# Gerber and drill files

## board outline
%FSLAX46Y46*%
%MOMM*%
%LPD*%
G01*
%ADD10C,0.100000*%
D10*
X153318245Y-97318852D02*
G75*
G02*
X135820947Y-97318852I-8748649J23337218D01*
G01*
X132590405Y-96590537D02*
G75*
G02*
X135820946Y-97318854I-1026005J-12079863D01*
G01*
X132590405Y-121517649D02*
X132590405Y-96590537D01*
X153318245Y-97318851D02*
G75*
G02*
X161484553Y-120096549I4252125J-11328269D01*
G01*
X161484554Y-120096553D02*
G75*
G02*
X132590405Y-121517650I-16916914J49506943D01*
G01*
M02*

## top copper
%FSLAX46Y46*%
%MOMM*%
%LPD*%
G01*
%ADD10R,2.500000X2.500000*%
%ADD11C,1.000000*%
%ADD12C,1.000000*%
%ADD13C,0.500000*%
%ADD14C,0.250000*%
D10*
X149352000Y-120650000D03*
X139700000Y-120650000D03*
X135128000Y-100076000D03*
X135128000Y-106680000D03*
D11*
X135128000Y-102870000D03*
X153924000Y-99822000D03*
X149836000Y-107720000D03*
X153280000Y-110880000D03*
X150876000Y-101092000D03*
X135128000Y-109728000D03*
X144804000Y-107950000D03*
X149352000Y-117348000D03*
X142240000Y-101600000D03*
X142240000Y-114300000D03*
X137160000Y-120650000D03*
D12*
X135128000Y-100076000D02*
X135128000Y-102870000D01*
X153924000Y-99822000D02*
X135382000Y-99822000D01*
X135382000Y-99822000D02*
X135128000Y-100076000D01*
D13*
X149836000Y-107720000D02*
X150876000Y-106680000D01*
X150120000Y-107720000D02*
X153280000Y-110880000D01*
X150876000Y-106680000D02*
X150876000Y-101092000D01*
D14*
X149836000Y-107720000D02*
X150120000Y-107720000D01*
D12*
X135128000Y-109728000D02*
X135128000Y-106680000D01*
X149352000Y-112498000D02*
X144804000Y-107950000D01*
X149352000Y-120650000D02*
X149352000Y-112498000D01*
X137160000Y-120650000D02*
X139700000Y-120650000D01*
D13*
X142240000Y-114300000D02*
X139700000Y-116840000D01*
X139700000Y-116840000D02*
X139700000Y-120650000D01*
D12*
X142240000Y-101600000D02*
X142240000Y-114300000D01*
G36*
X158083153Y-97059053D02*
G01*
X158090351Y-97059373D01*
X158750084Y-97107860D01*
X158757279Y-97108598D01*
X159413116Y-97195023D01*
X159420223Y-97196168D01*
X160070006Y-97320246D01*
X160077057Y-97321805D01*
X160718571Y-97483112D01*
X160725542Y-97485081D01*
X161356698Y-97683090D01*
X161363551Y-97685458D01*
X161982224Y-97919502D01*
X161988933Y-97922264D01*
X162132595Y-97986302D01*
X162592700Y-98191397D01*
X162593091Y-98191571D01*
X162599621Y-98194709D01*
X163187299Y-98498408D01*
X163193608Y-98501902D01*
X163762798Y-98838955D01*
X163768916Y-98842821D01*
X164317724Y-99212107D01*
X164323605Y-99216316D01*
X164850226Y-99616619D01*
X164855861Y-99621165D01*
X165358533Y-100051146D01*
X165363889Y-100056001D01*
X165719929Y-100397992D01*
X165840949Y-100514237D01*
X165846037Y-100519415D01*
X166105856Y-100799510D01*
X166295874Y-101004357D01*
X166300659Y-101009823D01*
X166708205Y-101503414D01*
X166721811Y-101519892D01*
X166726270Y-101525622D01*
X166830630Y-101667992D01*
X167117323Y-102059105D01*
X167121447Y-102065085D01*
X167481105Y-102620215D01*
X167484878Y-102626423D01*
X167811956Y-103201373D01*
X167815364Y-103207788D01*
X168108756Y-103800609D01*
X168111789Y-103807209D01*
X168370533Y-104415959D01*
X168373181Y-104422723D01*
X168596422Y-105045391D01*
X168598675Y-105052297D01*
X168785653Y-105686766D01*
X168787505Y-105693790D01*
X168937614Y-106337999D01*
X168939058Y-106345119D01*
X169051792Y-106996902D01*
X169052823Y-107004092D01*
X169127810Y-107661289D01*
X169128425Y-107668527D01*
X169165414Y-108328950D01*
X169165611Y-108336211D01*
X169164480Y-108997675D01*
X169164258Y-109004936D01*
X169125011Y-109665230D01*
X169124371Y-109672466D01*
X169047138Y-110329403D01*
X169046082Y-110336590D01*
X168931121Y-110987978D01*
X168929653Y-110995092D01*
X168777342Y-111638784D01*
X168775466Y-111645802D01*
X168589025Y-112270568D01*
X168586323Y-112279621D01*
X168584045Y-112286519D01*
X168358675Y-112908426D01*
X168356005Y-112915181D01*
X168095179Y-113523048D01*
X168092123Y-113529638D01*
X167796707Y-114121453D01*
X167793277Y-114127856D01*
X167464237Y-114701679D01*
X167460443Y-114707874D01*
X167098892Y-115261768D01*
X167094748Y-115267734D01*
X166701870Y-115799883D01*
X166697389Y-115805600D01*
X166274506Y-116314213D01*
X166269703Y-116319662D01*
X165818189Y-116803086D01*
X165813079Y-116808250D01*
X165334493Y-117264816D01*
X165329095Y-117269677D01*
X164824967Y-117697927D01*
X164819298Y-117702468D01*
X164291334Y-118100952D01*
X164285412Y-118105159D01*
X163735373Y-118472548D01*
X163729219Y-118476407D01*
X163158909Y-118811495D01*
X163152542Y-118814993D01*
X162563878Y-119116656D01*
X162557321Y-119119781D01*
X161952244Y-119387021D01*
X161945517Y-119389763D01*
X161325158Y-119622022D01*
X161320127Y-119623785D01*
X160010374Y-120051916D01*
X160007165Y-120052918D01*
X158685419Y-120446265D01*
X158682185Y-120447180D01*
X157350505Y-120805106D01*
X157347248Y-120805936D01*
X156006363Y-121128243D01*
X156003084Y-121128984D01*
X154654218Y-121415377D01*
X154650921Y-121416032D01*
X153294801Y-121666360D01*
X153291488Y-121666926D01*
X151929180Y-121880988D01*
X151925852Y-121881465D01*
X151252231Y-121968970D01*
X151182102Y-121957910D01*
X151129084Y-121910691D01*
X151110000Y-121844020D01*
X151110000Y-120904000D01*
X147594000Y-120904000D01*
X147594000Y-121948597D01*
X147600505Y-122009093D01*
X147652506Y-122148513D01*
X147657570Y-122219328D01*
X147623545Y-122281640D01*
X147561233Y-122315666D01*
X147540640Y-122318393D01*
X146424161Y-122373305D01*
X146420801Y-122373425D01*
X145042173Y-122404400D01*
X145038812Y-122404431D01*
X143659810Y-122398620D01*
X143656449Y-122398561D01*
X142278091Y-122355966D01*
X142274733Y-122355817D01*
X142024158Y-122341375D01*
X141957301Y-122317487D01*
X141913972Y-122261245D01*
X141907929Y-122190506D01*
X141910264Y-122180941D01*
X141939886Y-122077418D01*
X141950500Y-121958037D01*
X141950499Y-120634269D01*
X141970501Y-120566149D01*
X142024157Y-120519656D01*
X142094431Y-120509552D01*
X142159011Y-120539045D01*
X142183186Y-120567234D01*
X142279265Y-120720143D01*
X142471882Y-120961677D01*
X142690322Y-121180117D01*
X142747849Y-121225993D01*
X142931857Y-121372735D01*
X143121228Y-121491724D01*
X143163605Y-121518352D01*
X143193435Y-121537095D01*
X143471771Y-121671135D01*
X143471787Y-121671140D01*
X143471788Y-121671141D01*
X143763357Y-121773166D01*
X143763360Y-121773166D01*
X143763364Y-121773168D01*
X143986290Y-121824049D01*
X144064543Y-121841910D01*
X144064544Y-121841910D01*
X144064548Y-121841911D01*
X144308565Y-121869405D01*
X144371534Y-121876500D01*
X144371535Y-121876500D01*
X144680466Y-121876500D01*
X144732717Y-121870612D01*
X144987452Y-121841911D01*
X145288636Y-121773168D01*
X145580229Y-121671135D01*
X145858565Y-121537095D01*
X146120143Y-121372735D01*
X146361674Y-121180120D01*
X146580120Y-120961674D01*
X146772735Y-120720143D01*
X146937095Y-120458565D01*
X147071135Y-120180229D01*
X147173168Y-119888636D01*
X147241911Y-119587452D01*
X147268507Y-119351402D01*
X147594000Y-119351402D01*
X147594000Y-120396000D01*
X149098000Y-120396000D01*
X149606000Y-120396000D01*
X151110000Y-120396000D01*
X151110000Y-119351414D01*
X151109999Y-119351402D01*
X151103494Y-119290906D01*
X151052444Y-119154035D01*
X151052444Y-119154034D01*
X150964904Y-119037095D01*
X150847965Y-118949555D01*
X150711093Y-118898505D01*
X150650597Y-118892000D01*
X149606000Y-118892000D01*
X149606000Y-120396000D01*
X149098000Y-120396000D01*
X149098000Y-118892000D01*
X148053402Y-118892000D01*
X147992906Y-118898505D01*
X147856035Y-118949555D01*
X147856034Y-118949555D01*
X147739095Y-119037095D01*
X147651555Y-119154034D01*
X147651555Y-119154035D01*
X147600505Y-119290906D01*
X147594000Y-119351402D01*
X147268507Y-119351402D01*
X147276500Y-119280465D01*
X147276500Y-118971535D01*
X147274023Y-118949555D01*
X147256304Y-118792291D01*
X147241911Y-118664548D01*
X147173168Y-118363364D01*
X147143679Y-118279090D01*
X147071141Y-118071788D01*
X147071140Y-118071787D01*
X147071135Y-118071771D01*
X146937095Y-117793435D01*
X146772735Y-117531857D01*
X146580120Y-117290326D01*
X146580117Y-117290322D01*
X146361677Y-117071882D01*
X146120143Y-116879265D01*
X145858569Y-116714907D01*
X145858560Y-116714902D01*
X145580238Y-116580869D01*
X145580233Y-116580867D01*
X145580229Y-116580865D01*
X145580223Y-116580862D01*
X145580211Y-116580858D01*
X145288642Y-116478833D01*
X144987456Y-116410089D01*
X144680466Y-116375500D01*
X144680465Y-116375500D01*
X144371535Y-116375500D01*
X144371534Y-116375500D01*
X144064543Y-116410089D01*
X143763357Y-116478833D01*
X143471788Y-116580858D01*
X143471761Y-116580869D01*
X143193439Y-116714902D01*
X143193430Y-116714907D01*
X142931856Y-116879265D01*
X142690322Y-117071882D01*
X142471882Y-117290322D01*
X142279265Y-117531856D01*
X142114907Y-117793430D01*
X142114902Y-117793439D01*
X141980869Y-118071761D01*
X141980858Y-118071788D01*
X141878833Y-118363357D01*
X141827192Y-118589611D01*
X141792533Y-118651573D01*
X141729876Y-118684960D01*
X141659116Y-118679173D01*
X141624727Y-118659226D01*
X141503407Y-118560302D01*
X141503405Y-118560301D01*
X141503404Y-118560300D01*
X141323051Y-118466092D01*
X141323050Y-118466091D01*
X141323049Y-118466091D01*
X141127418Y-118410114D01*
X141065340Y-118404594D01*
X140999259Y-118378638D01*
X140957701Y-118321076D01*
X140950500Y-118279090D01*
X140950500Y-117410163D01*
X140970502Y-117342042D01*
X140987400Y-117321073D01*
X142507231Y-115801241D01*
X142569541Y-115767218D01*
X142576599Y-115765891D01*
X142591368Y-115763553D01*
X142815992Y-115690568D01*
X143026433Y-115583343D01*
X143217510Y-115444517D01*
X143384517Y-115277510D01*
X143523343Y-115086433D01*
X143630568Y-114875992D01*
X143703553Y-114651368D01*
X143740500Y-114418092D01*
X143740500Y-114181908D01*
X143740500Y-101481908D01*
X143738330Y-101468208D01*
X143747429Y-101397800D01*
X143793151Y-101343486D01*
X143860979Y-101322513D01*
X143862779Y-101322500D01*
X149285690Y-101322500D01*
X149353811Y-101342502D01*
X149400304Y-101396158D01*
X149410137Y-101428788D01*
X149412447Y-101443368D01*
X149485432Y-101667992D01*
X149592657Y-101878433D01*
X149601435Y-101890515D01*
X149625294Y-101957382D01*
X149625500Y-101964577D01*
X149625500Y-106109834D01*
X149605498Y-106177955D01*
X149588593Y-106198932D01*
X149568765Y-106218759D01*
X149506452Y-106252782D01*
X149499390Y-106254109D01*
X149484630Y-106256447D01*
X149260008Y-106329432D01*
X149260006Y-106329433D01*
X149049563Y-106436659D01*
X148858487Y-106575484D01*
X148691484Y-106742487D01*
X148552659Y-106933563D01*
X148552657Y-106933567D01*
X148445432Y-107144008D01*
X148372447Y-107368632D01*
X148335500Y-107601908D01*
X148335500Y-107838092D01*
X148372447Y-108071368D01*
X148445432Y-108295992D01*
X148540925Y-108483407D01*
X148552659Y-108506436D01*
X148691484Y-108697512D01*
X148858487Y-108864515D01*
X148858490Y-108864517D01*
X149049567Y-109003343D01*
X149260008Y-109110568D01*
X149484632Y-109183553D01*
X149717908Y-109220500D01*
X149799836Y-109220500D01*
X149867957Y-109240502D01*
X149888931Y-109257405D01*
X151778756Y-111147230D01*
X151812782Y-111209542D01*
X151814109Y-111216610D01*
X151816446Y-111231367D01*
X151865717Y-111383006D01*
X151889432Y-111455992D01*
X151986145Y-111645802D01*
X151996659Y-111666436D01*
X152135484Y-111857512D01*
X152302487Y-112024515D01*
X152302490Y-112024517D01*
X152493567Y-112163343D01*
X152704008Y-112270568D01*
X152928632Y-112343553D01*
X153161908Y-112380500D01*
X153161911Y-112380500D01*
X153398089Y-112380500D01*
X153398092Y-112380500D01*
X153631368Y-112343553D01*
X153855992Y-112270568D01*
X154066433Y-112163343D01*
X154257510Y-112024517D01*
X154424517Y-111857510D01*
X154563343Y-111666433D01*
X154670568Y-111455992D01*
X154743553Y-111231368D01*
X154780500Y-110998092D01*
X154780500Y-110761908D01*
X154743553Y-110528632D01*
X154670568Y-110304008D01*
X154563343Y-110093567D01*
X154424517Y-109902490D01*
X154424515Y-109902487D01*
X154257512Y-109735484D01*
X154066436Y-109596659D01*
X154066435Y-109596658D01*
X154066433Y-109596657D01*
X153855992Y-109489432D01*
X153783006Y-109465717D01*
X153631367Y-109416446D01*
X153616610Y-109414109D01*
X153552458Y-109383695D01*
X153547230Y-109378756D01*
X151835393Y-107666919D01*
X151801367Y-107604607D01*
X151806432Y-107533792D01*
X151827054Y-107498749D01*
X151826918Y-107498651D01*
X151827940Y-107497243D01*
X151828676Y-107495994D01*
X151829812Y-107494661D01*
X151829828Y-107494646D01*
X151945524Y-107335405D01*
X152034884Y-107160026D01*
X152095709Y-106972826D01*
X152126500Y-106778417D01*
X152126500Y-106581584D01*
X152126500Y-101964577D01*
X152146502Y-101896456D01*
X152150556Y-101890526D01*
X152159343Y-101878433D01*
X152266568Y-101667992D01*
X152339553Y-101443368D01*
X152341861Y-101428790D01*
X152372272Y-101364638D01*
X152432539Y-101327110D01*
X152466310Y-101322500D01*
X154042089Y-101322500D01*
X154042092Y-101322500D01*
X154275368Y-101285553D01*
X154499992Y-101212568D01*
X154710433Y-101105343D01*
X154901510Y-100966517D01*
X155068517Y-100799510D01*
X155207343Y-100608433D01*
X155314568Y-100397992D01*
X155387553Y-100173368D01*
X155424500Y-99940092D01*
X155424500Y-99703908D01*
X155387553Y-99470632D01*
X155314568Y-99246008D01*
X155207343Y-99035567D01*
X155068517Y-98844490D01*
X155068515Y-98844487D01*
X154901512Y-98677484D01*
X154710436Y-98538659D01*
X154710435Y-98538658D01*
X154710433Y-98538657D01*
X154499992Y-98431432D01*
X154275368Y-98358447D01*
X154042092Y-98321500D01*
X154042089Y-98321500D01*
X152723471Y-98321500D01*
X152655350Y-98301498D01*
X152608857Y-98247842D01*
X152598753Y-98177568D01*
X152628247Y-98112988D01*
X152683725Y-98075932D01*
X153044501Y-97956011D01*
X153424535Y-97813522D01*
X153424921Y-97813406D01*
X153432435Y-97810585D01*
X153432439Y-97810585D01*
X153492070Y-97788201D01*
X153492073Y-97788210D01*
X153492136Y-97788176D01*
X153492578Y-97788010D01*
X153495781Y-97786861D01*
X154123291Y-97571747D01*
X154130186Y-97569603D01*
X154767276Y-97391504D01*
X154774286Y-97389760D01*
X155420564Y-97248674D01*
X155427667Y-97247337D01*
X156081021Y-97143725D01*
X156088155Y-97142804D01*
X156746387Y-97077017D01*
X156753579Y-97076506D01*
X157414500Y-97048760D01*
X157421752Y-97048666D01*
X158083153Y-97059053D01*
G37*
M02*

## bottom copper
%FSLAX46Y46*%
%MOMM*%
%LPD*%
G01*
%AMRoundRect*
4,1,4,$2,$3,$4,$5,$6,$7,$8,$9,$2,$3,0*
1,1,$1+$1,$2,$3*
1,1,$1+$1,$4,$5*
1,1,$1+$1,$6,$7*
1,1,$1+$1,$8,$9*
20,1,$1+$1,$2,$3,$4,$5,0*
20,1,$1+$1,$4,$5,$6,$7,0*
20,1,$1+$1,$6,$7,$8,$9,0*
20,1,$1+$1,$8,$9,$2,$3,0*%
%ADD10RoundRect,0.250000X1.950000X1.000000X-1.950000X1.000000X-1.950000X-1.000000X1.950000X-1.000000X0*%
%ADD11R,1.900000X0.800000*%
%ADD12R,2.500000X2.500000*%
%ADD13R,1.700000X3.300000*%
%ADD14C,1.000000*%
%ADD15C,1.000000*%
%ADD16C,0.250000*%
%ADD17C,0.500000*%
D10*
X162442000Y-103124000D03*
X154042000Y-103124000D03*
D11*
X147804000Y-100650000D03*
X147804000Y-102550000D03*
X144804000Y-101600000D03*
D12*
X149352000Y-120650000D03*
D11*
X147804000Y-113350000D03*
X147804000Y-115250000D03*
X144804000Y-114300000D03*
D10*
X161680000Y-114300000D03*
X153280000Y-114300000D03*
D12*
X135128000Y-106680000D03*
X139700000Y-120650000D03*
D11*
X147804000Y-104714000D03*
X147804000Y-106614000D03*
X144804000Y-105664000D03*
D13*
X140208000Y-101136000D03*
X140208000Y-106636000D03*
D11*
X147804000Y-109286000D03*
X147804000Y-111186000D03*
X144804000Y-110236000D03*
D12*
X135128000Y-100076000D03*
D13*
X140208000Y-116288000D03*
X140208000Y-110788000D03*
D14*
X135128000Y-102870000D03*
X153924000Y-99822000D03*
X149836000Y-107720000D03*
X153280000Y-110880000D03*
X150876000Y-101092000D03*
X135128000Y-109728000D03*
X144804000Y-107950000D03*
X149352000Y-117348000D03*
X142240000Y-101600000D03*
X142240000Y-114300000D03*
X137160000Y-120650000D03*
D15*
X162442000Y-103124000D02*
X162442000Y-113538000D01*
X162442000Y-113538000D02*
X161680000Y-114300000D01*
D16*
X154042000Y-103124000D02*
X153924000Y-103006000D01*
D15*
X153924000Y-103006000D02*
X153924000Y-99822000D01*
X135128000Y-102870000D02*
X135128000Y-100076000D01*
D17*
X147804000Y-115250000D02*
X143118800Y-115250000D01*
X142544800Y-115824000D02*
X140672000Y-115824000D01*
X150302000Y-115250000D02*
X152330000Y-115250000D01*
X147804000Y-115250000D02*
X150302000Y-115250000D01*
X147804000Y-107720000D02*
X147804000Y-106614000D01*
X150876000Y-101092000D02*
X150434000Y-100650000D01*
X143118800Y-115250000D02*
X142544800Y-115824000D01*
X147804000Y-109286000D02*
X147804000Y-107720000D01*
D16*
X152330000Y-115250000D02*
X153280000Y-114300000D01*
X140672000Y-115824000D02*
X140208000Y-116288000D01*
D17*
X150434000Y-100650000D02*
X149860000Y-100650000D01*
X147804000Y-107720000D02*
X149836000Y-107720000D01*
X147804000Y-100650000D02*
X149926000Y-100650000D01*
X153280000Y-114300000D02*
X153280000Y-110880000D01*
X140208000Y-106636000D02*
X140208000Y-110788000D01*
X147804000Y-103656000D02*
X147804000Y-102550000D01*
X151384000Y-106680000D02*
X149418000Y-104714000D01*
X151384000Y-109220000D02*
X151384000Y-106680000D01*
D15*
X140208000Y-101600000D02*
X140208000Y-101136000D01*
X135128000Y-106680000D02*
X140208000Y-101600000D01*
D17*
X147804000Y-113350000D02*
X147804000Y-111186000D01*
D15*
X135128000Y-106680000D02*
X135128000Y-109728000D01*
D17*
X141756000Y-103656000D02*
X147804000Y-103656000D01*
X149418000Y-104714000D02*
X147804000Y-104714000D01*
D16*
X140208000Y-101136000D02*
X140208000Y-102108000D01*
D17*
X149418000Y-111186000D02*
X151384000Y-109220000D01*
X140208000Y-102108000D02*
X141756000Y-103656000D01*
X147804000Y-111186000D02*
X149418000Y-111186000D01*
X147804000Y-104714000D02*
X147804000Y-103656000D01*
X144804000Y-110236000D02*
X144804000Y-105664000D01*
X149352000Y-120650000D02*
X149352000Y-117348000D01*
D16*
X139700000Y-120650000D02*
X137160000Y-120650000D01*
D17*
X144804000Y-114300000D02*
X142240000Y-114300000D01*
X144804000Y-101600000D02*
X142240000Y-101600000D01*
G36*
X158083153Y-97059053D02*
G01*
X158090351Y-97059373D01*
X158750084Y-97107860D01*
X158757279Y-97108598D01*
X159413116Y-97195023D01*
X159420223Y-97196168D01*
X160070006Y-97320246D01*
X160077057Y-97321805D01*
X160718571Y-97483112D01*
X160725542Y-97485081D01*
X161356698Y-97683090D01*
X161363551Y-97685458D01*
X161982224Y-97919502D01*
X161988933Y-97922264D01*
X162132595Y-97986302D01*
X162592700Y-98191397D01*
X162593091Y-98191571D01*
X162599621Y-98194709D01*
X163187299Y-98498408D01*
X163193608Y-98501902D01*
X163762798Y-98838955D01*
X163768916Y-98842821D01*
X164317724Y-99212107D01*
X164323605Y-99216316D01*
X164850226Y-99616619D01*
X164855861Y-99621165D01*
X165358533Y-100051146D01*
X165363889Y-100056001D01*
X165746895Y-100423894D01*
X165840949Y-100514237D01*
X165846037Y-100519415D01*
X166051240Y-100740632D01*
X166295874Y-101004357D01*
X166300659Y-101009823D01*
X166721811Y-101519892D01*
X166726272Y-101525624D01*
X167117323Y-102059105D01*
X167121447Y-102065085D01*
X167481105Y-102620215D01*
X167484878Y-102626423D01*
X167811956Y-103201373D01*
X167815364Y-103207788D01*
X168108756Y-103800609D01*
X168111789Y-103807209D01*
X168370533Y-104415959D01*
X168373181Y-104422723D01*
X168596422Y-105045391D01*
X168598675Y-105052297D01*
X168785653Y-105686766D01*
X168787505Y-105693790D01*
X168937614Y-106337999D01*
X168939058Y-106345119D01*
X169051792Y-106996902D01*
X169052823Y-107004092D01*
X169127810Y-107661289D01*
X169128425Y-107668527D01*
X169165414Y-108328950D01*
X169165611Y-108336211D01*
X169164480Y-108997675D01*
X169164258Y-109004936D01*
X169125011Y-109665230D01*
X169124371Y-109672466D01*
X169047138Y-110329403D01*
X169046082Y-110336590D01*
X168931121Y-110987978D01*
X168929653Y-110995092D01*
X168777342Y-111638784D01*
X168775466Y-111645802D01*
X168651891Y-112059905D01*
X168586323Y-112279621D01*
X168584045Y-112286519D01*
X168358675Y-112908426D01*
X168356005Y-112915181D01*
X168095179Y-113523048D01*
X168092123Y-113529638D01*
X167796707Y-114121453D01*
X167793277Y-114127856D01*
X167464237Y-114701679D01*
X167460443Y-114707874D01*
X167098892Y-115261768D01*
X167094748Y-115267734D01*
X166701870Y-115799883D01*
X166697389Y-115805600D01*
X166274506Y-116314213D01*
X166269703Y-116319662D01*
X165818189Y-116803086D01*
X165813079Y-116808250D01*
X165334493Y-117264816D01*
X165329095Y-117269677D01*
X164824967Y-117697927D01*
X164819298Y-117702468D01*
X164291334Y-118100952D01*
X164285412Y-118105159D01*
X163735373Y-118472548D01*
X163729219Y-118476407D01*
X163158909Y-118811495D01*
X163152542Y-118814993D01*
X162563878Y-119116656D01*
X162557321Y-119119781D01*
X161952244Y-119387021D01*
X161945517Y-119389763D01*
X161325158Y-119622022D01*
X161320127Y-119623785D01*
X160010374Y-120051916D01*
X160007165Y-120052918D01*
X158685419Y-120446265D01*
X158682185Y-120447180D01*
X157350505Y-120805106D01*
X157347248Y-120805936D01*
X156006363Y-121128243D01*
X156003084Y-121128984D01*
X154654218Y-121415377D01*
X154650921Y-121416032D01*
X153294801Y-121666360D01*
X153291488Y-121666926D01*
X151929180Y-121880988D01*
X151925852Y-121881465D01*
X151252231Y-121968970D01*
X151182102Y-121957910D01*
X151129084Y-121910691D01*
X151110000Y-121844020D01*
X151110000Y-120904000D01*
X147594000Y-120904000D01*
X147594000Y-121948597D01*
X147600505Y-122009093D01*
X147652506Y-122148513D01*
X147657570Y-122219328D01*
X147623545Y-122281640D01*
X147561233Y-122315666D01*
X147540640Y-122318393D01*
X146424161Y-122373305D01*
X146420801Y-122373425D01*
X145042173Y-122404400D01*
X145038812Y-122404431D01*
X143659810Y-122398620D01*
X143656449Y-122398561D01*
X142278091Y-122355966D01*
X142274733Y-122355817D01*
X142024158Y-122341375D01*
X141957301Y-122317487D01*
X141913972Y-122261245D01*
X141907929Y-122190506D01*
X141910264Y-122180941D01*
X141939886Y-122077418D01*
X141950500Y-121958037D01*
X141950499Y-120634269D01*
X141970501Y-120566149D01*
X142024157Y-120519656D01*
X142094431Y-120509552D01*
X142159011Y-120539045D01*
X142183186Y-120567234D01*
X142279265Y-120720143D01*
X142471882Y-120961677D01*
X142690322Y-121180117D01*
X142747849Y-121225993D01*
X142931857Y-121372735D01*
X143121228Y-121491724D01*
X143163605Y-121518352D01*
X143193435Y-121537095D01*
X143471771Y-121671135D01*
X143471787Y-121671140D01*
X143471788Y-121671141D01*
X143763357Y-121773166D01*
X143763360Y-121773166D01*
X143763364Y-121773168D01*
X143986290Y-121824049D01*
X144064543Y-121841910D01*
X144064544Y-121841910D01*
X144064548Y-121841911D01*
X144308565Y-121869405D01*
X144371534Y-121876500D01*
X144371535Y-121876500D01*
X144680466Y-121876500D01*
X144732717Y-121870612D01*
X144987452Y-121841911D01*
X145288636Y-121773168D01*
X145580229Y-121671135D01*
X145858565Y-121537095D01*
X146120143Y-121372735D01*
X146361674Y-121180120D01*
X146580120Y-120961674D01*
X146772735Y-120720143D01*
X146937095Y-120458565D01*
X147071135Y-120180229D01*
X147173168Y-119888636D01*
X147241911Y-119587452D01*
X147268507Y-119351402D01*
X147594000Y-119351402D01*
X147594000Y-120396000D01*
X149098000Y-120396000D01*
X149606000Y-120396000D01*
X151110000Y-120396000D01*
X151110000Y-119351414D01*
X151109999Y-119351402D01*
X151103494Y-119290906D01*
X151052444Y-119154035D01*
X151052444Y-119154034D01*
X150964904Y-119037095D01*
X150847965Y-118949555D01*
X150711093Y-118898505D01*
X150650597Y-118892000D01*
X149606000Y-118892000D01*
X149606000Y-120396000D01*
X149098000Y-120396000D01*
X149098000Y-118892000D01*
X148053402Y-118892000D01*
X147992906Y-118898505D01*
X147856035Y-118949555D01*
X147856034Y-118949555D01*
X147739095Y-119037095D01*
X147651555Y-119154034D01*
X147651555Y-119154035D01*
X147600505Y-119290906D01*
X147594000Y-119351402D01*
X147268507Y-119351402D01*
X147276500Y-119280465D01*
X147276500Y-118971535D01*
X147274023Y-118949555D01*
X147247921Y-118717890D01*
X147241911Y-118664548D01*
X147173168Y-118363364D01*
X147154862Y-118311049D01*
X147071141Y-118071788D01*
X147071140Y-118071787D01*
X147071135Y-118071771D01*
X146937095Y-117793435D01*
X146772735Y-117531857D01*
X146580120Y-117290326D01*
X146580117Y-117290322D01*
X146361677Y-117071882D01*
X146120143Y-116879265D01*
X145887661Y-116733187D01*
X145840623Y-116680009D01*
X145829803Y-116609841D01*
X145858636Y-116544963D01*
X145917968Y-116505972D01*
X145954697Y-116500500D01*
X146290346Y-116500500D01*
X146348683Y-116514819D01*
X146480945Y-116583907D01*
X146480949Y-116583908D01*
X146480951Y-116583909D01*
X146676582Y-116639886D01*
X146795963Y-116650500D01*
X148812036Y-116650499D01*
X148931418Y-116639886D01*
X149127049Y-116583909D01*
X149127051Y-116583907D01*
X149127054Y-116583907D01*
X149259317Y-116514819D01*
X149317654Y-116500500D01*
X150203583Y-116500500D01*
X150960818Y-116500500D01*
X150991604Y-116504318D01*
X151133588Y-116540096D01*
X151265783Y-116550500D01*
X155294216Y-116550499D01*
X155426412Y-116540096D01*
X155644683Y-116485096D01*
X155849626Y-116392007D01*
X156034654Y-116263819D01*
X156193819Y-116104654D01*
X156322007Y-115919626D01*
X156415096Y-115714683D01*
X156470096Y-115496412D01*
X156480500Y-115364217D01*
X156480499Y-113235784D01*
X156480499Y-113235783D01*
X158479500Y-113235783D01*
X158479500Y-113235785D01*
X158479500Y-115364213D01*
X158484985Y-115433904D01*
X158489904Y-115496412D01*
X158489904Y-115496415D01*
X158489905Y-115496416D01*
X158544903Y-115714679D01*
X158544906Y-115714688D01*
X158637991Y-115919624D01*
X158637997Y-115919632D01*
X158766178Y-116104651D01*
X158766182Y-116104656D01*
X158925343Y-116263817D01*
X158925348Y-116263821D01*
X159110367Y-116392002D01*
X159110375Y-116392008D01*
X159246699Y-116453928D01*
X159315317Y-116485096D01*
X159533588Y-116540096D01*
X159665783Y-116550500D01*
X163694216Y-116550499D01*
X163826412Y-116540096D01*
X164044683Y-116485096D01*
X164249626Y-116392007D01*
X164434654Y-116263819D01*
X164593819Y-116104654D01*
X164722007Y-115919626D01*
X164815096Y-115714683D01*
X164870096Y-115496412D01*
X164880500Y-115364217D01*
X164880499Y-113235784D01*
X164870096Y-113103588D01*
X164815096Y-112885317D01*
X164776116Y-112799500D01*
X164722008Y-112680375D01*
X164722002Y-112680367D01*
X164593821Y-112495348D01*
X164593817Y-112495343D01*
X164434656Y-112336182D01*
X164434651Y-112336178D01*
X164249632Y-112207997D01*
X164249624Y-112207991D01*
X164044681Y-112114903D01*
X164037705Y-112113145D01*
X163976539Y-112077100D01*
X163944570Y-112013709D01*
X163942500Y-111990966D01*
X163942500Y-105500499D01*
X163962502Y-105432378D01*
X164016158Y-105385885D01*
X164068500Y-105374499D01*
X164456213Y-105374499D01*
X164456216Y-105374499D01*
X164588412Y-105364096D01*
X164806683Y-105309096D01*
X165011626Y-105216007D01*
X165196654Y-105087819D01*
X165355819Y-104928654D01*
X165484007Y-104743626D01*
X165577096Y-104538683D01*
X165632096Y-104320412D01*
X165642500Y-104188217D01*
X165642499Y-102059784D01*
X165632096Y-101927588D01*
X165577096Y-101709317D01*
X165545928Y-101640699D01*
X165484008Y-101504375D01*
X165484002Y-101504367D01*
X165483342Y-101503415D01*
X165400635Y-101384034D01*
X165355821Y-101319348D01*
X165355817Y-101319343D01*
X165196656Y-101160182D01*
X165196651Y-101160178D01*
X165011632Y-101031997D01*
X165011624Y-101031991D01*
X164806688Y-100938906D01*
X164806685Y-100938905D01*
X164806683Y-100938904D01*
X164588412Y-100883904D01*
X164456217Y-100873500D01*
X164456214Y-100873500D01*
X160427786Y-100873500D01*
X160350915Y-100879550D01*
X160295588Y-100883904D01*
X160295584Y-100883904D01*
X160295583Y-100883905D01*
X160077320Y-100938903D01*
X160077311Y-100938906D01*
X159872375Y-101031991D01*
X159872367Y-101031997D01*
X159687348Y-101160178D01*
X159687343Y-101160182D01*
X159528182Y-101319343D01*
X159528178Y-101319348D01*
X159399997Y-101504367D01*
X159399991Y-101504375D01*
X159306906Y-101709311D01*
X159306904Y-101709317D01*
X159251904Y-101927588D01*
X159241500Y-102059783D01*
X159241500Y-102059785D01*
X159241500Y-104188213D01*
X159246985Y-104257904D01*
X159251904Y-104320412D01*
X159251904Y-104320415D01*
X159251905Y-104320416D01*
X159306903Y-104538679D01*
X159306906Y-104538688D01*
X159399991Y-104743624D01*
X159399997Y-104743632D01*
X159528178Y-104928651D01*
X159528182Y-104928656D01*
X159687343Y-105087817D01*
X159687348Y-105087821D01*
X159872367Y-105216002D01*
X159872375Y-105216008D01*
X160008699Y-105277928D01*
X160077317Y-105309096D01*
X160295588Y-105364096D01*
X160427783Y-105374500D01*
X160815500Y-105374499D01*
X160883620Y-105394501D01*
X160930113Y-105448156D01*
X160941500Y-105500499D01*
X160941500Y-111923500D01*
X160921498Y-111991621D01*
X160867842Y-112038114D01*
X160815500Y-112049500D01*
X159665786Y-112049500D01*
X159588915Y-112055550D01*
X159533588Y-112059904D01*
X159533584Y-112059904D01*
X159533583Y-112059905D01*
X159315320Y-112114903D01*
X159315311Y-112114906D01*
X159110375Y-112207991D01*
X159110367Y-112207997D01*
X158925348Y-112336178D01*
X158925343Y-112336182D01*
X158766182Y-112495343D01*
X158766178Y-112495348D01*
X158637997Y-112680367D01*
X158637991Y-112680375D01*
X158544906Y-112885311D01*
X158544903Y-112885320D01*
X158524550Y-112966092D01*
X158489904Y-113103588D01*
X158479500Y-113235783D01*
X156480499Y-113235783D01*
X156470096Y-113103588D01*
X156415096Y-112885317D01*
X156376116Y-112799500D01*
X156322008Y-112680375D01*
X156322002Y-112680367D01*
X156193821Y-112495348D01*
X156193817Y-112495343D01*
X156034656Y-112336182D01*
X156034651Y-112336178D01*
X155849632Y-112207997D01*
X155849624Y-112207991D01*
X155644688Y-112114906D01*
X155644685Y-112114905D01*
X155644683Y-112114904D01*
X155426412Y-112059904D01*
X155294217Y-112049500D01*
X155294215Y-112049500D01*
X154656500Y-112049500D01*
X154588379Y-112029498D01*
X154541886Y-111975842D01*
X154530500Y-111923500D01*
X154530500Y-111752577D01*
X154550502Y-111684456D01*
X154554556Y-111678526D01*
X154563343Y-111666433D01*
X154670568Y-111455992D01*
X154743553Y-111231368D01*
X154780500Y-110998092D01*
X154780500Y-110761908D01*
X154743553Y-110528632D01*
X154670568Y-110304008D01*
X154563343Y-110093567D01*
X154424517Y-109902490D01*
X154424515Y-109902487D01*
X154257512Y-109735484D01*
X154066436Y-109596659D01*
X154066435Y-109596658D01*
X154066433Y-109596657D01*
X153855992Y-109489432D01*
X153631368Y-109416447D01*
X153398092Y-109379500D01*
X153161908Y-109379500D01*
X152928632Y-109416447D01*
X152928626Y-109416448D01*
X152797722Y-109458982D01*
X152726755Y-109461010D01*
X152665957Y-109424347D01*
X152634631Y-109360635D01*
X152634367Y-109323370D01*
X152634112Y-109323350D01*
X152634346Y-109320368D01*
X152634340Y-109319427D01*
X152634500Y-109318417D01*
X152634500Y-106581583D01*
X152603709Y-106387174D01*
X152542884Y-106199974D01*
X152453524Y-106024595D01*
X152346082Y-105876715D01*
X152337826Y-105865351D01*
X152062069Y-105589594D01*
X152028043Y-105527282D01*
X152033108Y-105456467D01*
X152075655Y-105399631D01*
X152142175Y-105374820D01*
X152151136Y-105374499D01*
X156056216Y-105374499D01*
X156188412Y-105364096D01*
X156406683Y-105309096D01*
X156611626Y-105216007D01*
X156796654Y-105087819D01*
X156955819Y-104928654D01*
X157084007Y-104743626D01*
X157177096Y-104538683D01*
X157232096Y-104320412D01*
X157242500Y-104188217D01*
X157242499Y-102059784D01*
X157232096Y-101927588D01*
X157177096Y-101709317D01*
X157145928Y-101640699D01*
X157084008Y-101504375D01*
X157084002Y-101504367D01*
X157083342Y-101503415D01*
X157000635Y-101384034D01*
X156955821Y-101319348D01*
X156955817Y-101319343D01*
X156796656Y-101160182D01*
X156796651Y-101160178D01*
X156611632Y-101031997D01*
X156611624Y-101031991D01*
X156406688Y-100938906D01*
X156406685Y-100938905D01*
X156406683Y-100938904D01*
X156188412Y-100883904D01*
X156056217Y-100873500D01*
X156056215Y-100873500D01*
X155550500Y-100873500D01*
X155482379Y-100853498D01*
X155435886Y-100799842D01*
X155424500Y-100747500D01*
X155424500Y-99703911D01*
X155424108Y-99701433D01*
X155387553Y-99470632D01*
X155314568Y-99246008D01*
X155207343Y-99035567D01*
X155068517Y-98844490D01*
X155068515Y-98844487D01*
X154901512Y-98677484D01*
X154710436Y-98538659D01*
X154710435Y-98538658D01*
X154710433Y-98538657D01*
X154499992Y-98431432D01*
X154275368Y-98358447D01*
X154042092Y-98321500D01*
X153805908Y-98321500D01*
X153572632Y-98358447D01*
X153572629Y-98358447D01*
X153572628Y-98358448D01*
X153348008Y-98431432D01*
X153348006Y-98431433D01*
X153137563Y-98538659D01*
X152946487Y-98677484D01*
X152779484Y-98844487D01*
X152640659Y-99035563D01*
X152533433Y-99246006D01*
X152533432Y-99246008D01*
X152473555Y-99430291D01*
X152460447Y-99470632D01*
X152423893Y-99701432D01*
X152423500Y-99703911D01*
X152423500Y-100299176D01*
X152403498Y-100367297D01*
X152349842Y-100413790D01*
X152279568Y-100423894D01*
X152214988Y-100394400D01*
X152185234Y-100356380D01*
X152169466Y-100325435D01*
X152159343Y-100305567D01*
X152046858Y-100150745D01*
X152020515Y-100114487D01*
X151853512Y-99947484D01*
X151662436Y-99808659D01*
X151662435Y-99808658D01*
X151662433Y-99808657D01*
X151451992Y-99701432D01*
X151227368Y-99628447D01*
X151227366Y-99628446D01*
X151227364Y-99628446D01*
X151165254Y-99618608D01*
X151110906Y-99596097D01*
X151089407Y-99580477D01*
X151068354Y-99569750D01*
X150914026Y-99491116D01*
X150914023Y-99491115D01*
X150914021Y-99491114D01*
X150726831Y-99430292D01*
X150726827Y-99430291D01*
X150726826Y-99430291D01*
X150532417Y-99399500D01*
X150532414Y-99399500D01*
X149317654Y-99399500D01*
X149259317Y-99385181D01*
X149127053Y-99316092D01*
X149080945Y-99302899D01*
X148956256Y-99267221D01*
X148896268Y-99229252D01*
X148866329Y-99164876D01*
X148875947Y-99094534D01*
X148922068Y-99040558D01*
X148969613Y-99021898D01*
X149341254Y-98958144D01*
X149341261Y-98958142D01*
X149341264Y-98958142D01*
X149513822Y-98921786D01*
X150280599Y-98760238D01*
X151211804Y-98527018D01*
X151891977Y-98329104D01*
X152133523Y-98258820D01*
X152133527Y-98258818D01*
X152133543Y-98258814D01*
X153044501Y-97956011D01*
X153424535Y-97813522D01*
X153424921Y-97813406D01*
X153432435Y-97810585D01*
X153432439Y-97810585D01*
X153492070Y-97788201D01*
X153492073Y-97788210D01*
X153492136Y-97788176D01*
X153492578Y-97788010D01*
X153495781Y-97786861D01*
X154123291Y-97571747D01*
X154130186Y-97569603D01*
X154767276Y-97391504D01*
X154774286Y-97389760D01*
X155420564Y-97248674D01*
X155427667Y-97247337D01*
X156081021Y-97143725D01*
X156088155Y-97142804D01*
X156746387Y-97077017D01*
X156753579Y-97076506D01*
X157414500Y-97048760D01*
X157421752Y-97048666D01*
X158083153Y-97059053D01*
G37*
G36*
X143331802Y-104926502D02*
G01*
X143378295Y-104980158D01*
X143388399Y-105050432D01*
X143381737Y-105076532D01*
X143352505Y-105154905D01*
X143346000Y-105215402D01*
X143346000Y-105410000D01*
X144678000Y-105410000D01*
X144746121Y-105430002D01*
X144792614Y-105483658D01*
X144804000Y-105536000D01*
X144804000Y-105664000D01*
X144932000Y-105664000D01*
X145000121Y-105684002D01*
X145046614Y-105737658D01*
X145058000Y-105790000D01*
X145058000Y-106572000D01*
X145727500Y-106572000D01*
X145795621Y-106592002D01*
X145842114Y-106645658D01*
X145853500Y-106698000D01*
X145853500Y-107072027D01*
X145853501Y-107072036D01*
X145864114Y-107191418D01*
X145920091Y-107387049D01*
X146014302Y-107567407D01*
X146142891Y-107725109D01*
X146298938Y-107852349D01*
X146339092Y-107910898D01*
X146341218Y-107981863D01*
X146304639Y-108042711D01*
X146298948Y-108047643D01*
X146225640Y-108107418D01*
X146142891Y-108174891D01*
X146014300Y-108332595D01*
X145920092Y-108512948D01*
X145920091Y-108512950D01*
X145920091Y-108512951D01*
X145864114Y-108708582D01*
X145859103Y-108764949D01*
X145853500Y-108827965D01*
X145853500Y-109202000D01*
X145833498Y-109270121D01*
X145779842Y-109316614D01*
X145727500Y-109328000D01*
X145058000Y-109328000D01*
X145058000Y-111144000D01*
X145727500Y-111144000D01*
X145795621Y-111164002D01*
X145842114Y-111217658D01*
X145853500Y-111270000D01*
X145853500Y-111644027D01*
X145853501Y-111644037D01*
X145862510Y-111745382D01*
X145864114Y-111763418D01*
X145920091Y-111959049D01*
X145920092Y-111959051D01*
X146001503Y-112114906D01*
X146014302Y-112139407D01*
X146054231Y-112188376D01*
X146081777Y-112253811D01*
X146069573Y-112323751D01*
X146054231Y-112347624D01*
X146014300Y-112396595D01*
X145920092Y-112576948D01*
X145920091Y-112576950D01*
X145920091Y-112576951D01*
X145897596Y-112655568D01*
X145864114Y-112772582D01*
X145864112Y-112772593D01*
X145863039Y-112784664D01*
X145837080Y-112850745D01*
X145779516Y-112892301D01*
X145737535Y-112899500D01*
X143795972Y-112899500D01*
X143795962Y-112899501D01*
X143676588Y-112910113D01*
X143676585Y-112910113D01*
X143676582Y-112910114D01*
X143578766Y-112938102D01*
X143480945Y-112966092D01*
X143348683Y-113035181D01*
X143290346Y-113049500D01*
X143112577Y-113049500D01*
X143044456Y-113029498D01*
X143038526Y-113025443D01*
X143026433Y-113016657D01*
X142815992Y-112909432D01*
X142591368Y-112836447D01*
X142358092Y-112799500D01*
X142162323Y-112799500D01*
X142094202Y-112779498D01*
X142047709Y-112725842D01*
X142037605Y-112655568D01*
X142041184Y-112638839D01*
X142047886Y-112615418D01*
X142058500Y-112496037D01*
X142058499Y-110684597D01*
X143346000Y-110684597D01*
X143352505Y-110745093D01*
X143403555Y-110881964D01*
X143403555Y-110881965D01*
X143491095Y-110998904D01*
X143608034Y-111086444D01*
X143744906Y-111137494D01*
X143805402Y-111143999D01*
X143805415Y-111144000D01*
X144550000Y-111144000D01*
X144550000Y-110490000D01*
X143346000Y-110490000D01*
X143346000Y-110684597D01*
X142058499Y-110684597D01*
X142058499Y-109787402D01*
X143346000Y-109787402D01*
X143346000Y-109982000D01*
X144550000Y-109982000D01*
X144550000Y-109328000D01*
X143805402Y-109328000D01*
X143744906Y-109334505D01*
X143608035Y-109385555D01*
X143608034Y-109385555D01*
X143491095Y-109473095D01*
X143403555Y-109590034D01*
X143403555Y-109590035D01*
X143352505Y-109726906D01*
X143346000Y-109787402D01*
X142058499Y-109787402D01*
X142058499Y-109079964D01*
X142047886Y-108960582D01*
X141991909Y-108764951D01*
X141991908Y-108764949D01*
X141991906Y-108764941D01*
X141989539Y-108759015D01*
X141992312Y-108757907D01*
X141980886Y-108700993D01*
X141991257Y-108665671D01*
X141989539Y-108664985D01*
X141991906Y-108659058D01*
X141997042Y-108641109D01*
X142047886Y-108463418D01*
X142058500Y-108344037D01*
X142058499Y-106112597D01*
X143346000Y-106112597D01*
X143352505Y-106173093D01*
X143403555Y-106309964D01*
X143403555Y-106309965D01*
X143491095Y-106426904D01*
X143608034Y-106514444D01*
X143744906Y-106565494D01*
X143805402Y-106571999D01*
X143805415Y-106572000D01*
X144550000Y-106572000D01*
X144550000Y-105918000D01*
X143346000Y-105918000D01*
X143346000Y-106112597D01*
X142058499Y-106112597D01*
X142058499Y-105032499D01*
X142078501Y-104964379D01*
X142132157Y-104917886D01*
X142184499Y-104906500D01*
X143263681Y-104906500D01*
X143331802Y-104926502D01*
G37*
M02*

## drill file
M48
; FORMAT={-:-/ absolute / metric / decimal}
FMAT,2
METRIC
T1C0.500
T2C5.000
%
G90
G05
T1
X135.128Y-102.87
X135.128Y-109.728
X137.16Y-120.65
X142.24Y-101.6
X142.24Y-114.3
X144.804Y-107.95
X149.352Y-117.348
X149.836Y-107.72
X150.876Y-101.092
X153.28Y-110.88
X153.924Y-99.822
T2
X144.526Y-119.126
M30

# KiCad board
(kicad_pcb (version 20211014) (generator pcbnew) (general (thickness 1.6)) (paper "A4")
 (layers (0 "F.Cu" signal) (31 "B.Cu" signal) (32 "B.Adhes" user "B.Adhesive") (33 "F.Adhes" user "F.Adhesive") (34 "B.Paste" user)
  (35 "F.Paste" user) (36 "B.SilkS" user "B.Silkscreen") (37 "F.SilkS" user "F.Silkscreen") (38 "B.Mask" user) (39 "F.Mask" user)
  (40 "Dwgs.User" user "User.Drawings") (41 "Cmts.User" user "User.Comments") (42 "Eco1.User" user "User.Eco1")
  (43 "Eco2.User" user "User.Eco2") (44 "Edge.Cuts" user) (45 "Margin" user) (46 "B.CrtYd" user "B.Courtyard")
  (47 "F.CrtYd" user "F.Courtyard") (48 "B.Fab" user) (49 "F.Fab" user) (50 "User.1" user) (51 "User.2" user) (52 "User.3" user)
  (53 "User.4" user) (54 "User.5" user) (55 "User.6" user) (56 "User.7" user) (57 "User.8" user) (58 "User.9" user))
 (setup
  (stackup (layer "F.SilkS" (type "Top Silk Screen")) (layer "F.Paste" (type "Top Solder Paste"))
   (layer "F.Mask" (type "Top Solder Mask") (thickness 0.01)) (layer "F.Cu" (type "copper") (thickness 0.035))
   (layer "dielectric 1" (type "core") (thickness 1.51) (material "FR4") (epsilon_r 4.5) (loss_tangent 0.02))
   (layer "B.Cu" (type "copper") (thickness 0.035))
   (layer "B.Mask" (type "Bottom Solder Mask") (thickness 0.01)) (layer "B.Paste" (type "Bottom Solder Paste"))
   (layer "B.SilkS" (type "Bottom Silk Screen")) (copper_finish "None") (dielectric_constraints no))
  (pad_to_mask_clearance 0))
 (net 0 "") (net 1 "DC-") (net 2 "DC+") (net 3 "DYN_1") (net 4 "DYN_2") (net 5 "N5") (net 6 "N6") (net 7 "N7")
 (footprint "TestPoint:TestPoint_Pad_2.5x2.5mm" (layer "F.Cu") (at 149.352 120.65 90)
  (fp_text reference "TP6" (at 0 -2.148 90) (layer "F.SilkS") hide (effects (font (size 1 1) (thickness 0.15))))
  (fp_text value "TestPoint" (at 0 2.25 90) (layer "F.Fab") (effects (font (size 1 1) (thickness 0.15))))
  (pad "1" smd rect (at 0 0 90) (size 2.5 2.5) (layers "F.Cu" "F.Mask") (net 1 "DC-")))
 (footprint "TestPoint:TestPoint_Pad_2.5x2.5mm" (layer "F.Cu") (at 139.7 120.65 90)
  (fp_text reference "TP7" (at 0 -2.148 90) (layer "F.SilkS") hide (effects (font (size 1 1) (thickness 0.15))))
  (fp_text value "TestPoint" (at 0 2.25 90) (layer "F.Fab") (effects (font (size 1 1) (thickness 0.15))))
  (pad "1" smd rect (at 0 0 90) (size 2.5 2.5) (layers "F.Cu" "F.Mask") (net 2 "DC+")))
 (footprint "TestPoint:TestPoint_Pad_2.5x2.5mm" (layer "F.Cu") (at 135.128 100.076 90)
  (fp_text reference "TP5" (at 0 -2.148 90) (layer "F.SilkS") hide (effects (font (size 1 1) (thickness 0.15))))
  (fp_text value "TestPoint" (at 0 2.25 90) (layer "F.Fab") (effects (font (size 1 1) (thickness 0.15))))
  (pad "1" smd rect (at 0 0 90) (size 2.5 2.5) (layers "F.Cu" "F.Mask") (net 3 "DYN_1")))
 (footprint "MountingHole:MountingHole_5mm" (layer "F.Cu") (at 144.526 119.126)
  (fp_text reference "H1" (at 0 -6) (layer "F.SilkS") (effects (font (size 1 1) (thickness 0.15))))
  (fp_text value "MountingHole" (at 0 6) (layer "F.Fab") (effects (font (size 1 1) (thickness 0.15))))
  (pad "" np_thru_hole circle (at 0 0) (size 5 5) (drill 5) (layers *.Cu *.Mask)))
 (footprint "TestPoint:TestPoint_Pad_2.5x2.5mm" (layer "F.Cu") (at 135.128 106.68)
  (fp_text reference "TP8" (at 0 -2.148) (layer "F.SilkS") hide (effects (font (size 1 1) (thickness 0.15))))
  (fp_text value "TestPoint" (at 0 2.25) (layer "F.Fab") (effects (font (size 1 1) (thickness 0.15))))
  (pad "1" smd rect (at 0 0) (size 2.5 2.5) (layers "F.Cu" "F.Mask") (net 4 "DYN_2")))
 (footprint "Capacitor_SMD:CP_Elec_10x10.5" (layer "B.Cu") (at 158.242 103.124 180)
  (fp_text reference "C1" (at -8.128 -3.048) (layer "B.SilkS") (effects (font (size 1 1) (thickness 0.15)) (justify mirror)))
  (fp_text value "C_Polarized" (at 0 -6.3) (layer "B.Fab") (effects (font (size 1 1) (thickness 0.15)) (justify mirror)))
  (pad "1" smd roundrect (at -4.2 0 180) (size 4.4 2.5) (layers "B.Cu" "B.Paste" "B.Mask") (roundrect_rratio 0.1) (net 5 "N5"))
  (pad "2" smd roundrect (at 4.2 0 180) (size 4.4 2.5) (layers "B.Cu" "B.Paste" "B.Mask") (roundrect_rratio 0.1) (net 3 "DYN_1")))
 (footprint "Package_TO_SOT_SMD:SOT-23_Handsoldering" (layer "B.Cu") (at 146.304 101.6 180)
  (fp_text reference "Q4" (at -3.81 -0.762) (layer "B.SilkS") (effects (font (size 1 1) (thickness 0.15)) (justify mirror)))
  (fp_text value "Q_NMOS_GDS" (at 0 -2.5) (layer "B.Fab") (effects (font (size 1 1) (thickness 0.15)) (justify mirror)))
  (pad "1" smd rect (at -1.5 0.95 180) (size 1.9 0.8) (layers "B.Cu" "B.Paste" "B.Mask") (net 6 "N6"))
  (pad "2" smd rect (at -1.5 -0.95 180) (size 1.9 0.8) (layers "B.Cu" "B.Paste" "B.Mask") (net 4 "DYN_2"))
  (pad "3" smd rect (at 1.5 0 180) (size 1.9 0.8) (layers "B.Cu" "B.Paste" "B.Mask") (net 2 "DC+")))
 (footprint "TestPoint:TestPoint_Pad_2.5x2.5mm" (layer "B.Cu") (at 149.352 120.65 -90)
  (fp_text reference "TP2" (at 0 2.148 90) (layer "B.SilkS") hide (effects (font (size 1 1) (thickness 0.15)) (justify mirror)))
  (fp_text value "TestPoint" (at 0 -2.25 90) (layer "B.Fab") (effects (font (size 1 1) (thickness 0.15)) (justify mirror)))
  (pad "1" smd rect (at 0 0 270) (size 2.5 2.5) (layers "B.Cu" "B.Mask") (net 1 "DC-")))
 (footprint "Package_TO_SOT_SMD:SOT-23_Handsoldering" (layer "B.Cu") (at 146.304 114.3 180)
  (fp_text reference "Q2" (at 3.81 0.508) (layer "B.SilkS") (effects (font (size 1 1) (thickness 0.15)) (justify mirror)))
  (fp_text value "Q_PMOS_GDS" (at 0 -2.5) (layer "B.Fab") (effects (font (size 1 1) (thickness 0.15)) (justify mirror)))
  (pad "1" smd rect (at -1.5 0.95 180) (size 1.9 0.8) (layers "B.Cu" "B.Paste" "B.Mask") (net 4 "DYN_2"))
  (pad "2" smd rect (at -1.5 -0.95 180) (size 1.9 0.8) (layers "B.Cu" "B.Paste" "B.Mask") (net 6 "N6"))
  (pad "3" smd rect (at 1.5 0 180) (size 1.9 0.8) (layers "B.Cu" "B.Paste" "B.Mask") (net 2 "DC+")))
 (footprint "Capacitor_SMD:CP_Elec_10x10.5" (layer "B.Cu") (at 157.48 114.3 180)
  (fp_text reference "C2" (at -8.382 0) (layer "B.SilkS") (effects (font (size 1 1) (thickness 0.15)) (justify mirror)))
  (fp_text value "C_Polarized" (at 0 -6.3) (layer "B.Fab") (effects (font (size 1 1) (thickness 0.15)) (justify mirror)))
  (pad "1" smd roundrect (at -4.2 0 180) (size 4.4 2.5) (layers "B.Cu" "B.Paste" "B.Mask") (roundrect_rratio 0.1) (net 5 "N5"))
  (pad "2" smd roundrect (at 4.2 0 180) (size 4.4 2.5) (layers "B.Cu" "B.Paste" "B.Mask") (roundrect_rratio 0.1) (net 6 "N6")))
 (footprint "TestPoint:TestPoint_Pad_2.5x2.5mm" (layer "B.Cu") (at 135.128 106.68 180)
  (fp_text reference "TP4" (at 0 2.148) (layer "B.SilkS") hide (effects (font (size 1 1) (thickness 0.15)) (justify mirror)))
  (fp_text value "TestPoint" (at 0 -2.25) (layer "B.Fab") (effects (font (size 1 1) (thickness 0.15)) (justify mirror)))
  (pad "1" smd rect (at 0 0 180) (size 2.5 2.5) (layers "B.Cu" "B.Mask") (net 4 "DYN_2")))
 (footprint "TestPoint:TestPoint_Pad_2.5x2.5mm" (layer "B.Cu") (at 139.7 120.65 -90)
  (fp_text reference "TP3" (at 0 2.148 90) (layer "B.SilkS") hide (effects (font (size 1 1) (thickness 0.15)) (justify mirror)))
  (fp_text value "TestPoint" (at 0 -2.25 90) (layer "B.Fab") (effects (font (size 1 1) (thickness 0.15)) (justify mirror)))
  (pad "1" smd rect (at 0 0 270) (size 2.5 2.5) (layers "B.Cu" "B.Mask") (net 2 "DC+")))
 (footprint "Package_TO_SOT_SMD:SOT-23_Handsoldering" (layer "B.Cu") (at 146.304 105.664 180)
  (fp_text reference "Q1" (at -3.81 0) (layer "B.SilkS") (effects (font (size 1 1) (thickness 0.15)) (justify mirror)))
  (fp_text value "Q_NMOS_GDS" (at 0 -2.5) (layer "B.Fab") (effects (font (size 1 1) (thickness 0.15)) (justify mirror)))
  (pad "1" smd rect (at -1.5 0.95 180) (size 1.9 0.8) (layers "B.Cu" "B.Paste" "B.Mask") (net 4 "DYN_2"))
  (pad "2" smd rect (at -1.5 -0.95 180) (size 1.9 0.8) (layers "B.Cu" "B.Paste" "B.Mask") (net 6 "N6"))
  (pad "3" smd rect (at 1.5 0 180) (size 1.9 0.8) (layers "B.Cu" "B.Paste" "B.Mask") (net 1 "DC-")))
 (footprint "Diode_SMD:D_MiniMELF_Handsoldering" (layer "B.Cu") (at 140.208 103.886 -90)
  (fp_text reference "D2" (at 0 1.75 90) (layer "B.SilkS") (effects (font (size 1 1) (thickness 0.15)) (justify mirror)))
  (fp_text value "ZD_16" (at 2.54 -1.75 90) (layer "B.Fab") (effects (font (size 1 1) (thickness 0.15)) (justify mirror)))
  (pad "1" smd rect (at -2.75 0 270) (size 3.3 1.7) (layers "B.Cu" "B.Paste" "B.Mask") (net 4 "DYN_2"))
  (pad "2" smd rect (at 2.75 0 270) (size 3.3 1.7) (layers "B.Cu" "B.Paste" "B.Mask") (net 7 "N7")))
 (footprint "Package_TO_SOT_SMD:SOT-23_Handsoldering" (layer "B.Cu") (at 146.304 110.236 180)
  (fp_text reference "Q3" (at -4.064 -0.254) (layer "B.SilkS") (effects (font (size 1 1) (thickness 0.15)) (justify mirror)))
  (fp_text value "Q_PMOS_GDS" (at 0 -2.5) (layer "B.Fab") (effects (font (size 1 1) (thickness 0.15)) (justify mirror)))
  (pad "1" smd rect (at -1.5 0.95 180) (size 1.9 0.8) (layers "B.Cu" "B.Paste" "B.Mask") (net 6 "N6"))
  (pad "2" smd rect (at -1.5 -0.95 180) (size 1.9 0.8) (layers "B.Cu" "B.Paste" "B.Mask") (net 4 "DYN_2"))
  (pad "3" smd rect (at 1.5 0 180) (size 1.9 0.8) (layers "B.Cu" "B.Paste" "B.Mask") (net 1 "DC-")))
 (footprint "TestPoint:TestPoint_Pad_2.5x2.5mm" (layer "B.Cu") (at 135.128 100.076 -90)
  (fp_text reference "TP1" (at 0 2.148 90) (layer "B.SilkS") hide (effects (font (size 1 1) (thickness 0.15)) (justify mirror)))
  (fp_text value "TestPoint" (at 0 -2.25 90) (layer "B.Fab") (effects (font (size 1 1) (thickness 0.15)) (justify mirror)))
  (pad "1" smd rect (at 0 0 270) (size 2.5 2.5) (layers "B.Cu" "B.Mask") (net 3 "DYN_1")))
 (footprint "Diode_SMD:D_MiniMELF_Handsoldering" (layer "B.Cu") (at 140.208 113.538 90)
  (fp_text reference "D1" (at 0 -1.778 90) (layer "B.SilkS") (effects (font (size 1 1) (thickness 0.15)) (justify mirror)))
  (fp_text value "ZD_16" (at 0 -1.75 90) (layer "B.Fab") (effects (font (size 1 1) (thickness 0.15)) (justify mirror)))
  (pad "1" smd rect (at -2.75 0 90) (size 3.3 1.7) (layers "B.Cu" "B.Paste" "B.Mask") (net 6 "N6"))
  (pad "2" smd rect (at 2.75 0 90) (size 3.3 1.7) (layers "B.Cu" "B.Paste" "B.Mask") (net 7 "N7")))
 (gr_arc (start 153.318245 97.318852) (mid 144.569596 98.904808) (end 135.820947 97.318852) (layer "Edge.Cuts") (width 0.1))
 (gr_arc (start 132.590405 96.590537) (mid 134.230661 96.843868) (end 135.820947 97.318851) (layer "Edge.Cuts") (width 0.1))
 (gr_line (start 132.590405 121.517649) (end 132.590405 96.590537) (layer "Edge.Cuts") (width 0.1))
 (gr_arc (start 153.318245 97.318851) (mid 168.960475 104.563518) (end 161.484554 120.096553) (layer "Edge.Cuts") (width 0.1))
 (gr_arc (start 161.484554 120.096553) (mid 147.137657 122.843934) (end 132.590405 121.517649) (layer "Edge.Cuts") (width 0.1))
 (segment (start 162.442 103.124) (end 162.442 113.538) (width 1) (layer "B.Cu") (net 5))
 (segment (start 162.442 113.538) (end 161.68 114.3) (width 1) (layer "B.Cu") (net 5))
 (segment (start 135.128 100.076) (end 135.128 102.87) (width 1) (layer "F.Cu") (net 3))
 (segment (start 153.924 99.822) (end 135.382 99.822) (width 1) (layer "F.Cu") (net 3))
 (segment (start 135.382 99.822) (end 135.128 100.076) (width 1) (layer "F.Cu") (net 3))
 (via (at 135.128 102.87) (size 1) (drill 0.5) (layers "F.Cu" "B.Cu") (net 3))
 (via (at 153.924 99.822) (size 1) (drill 0.5) (layers "F.Cu" "B.Cu") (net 3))
 (segment (start 154.042 103.124) (end 153.924 103.006) (width 0.25) (layer "B.Cu") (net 3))
 (segment (start 153.924 103.006) (end 153.924 99.822) (width 1) (layer "B.Cu") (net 3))
 (segment (start 135.128 102.87) (end 135.128 100.076) (width 1) (layer "B.Cu") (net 3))
 (segment (start 149.836 107.72) (end 150.876 106.68) (width 0.5) (layer "F.Cu") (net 6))
 (segment (start 150.12 107.72) (end 153.28 110.88) (width 0.5) (layer "F.Cu") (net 6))
 (segment (start 150.876 106.68) (end 150.876 101.092) (width 0.5) (layer "F.Cu") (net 6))
 (segment (start 149.836 107.72) (end 150.12 107.72) (width 0.25) (layer "F.Cu") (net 6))
 (via (at 149.836 107.72) (size 1) (drill 0.5) (layers "F.Cu" "B.Cu") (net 6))
 (via (at 153.28 110.88) (size 1) (drill 0.5) (layers "F.Cu" "B.Cu") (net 6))
 (via (at 150.876 101.092) (size 1) (drill 0.5) (layers "F.Cu" "B.Cu") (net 6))
 (segment (start 147.804 115.25) (end 143.1188 115.25) (width 0.5) (layer "B.Cu") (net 6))
 (segment (start 142.5448 115.824) (end 140.672 115.824) (width 0.5) (layer "B.Cu") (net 6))
 (segment (start 150.302 115.25) (end 152.33 115.25) (width 0.5) (layer "B.Cu") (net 6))
 (segment (start 147.804 115.25) (end 150.302 115.25) (width 0.5) (layer "B.Cu") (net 6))
 (segment (start 147.804 107.72) (end 147.804 106.614) (width 0.5) (layer "B.Cu") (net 6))
 (segment (start 150.876 101.092) (end 150.434 100.65) (width 0.5) (layer "B.Cu") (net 6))
 (segment (start 143.1188 115.25) (end 142.5448 115.824) (width 0.5) (layer "B.Cu") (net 6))
 (segment (start 147.804 109.286) (end 147.804 107.72) (width 0.5) (layer "B.Cu") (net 6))
 (segment (start 152.33 115.25) (end 153.28 114.3) (width 0.25) (layer "B.Cu") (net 6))
 (segment (start 140.672 115.824) (end 140.208 116.288) (width 0.25) (layer "B.Cu") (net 6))
 (segment (start 150.434 100.65) (end 149.86 100.65) (width 0.5) (layer "B.Cu") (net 6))
 (segment (start 147.804 107.72) (end 149.836 107.72) (width 0.5) (layer "B.Cu") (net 6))
 (segment (start 147.804 100.65) (end 149.926 100.65) (width 0.5) (layer "B.Cu") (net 6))
 (segment (start 153.28 114.3) (end 153.28 110.88) (width 0.5) (layer "B.Cu") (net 6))
 (segment (start 140.208 106.636) (end 140.208 110.788) (width 0.5) (layer "B.Cu") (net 7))
 (segment (start 135.128 109.728) (end 135.128 106.68) (width 1) (layer "F.Cu") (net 4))
 (via (at 135.128 109.728) (size 1) (drill 0.5) (layers "F.Cu" "B.Cu") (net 4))
 (segment (start 147.804 103.656) (end 147.804 102.55) (width 0.5) (layer "B.Cu") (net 4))
 (segment (start 151.384 106.68) (end 149.418 104.714) (width 0.5) (layer "B.Cu") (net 4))
 (segment (start 151.384 109.22) (end 151.384 106.68) (width 0.5) (layer "B.Cu") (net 4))
 (segment (start 140.208 101.6) (end 140.208 101.136) (width 1) (layer "B.Cu") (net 4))
 (segment (start 135.128 106.68) (end 140.208 101.6) (width 1) (layer "B.Cu") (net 4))
 (segment (start 147.804 113.35) (end 147.804 111.186) (width 0.5) (layer "B.Cu") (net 4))
 (segment (start 135.128 106.68) (end 135.128 109.728) (width 1) (layer "B.Cu") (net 4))
 (segment (start 141.756 103.656) (end 147.804 103.656) (width 0.5) (layer "B.Cu") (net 4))
 (segment (start 149.418 104.714) (end 147.804 104.714) (width 0.5) (layer "B.Cu") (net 4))
 (segment (start 140.208 101.136) (end 140.208 102.108) (width 0.25) (layer "B.Cu") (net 4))
 (segment (start 149.418 111.186) (end 151.384 109.22) (width 0.5) (layer "B.Cu") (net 4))
 (segment (start 140.208 102.108) (end 141.756 103.656) (width 0.5) (layer "B.Cu") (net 4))
 (segment (start 147.804 111.186) (end 149.418 111.186) (width 0.5) (layer "B.Cu") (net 4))
 (segment (start 147.804 104.714) (end 147.804 103.656) (width 0.5) (layer "B.Cu") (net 4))
 (segment (start 149.352 112.498) (end 144.804 107.95) (width 1) (layer "F.Cu") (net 1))
 (segment (start 149.352 120.65) (end 149.352 112.498) (width 1) (layer "F.Cu") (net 1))
 (via (at 144.804 107.95) (size 1) (drill 0.5) (layers "F.Cu" "B.Cu") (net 1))
 (via (at 149.352 117.348) (size 1) (drill 0.5) (layers "F.Cu" "B.Cu") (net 1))
 (segment (start 144.804 110.236) (end 144.804 105.664) (width 0.5) (layer "B.Cu") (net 1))
 (segment (start 149.352 120.65) (end 149.352 117.348) (width 0.5) (layer "B.Cu") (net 1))
 (segment (start 137.16 120.65) (end 139.7 120.65) (width 1) (layer "F.Cu") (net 2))
 (segment (start 142.24 114.3) (end 139.7 116.84) (width 0.5) (layer "F.Cu") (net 2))
 (segment (start 139.7 116.84) (end 139.7 120.65) (width 0.5) (layer "F.Cu") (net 2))
 (segment (start 142.24 101.6) (end 142.24 114.3) (width 1) (layer "F.Cu") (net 2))
 (via (at 142.24 101.6) (size 1) (drill 0.5) (layers "F.Cu" "B.Cu") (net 2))
 (via (at 142.24 114.3) (size 1) (drill 0.5) (layers "F.Cu" "B.Cu") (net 2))
 (via (at 137.16 120.65) (size 1) (drill 0.5) (layers "F.Cu" "B.Cu") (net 2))
 (segment (start 139.7 120.65) (end 137.16 120.65) (width 0.25) (layer "B.Cu") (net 2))
 (segment (start 144.804 114.3) (end 142.24 114.3) (width 0.5) (layer "B.Cu") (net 2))
 (segment (start 144.804 101.6) (end 142.24 101.6) (width 0.5) (layer "B.Cu") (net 2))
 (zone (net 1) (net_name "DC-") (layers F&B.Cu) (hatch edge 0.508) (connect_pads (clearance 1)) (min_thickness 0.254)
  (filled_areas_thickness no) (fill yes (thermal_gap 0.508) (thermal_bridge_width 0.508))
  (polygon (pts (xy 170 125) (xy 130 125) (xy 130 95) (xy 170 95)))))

